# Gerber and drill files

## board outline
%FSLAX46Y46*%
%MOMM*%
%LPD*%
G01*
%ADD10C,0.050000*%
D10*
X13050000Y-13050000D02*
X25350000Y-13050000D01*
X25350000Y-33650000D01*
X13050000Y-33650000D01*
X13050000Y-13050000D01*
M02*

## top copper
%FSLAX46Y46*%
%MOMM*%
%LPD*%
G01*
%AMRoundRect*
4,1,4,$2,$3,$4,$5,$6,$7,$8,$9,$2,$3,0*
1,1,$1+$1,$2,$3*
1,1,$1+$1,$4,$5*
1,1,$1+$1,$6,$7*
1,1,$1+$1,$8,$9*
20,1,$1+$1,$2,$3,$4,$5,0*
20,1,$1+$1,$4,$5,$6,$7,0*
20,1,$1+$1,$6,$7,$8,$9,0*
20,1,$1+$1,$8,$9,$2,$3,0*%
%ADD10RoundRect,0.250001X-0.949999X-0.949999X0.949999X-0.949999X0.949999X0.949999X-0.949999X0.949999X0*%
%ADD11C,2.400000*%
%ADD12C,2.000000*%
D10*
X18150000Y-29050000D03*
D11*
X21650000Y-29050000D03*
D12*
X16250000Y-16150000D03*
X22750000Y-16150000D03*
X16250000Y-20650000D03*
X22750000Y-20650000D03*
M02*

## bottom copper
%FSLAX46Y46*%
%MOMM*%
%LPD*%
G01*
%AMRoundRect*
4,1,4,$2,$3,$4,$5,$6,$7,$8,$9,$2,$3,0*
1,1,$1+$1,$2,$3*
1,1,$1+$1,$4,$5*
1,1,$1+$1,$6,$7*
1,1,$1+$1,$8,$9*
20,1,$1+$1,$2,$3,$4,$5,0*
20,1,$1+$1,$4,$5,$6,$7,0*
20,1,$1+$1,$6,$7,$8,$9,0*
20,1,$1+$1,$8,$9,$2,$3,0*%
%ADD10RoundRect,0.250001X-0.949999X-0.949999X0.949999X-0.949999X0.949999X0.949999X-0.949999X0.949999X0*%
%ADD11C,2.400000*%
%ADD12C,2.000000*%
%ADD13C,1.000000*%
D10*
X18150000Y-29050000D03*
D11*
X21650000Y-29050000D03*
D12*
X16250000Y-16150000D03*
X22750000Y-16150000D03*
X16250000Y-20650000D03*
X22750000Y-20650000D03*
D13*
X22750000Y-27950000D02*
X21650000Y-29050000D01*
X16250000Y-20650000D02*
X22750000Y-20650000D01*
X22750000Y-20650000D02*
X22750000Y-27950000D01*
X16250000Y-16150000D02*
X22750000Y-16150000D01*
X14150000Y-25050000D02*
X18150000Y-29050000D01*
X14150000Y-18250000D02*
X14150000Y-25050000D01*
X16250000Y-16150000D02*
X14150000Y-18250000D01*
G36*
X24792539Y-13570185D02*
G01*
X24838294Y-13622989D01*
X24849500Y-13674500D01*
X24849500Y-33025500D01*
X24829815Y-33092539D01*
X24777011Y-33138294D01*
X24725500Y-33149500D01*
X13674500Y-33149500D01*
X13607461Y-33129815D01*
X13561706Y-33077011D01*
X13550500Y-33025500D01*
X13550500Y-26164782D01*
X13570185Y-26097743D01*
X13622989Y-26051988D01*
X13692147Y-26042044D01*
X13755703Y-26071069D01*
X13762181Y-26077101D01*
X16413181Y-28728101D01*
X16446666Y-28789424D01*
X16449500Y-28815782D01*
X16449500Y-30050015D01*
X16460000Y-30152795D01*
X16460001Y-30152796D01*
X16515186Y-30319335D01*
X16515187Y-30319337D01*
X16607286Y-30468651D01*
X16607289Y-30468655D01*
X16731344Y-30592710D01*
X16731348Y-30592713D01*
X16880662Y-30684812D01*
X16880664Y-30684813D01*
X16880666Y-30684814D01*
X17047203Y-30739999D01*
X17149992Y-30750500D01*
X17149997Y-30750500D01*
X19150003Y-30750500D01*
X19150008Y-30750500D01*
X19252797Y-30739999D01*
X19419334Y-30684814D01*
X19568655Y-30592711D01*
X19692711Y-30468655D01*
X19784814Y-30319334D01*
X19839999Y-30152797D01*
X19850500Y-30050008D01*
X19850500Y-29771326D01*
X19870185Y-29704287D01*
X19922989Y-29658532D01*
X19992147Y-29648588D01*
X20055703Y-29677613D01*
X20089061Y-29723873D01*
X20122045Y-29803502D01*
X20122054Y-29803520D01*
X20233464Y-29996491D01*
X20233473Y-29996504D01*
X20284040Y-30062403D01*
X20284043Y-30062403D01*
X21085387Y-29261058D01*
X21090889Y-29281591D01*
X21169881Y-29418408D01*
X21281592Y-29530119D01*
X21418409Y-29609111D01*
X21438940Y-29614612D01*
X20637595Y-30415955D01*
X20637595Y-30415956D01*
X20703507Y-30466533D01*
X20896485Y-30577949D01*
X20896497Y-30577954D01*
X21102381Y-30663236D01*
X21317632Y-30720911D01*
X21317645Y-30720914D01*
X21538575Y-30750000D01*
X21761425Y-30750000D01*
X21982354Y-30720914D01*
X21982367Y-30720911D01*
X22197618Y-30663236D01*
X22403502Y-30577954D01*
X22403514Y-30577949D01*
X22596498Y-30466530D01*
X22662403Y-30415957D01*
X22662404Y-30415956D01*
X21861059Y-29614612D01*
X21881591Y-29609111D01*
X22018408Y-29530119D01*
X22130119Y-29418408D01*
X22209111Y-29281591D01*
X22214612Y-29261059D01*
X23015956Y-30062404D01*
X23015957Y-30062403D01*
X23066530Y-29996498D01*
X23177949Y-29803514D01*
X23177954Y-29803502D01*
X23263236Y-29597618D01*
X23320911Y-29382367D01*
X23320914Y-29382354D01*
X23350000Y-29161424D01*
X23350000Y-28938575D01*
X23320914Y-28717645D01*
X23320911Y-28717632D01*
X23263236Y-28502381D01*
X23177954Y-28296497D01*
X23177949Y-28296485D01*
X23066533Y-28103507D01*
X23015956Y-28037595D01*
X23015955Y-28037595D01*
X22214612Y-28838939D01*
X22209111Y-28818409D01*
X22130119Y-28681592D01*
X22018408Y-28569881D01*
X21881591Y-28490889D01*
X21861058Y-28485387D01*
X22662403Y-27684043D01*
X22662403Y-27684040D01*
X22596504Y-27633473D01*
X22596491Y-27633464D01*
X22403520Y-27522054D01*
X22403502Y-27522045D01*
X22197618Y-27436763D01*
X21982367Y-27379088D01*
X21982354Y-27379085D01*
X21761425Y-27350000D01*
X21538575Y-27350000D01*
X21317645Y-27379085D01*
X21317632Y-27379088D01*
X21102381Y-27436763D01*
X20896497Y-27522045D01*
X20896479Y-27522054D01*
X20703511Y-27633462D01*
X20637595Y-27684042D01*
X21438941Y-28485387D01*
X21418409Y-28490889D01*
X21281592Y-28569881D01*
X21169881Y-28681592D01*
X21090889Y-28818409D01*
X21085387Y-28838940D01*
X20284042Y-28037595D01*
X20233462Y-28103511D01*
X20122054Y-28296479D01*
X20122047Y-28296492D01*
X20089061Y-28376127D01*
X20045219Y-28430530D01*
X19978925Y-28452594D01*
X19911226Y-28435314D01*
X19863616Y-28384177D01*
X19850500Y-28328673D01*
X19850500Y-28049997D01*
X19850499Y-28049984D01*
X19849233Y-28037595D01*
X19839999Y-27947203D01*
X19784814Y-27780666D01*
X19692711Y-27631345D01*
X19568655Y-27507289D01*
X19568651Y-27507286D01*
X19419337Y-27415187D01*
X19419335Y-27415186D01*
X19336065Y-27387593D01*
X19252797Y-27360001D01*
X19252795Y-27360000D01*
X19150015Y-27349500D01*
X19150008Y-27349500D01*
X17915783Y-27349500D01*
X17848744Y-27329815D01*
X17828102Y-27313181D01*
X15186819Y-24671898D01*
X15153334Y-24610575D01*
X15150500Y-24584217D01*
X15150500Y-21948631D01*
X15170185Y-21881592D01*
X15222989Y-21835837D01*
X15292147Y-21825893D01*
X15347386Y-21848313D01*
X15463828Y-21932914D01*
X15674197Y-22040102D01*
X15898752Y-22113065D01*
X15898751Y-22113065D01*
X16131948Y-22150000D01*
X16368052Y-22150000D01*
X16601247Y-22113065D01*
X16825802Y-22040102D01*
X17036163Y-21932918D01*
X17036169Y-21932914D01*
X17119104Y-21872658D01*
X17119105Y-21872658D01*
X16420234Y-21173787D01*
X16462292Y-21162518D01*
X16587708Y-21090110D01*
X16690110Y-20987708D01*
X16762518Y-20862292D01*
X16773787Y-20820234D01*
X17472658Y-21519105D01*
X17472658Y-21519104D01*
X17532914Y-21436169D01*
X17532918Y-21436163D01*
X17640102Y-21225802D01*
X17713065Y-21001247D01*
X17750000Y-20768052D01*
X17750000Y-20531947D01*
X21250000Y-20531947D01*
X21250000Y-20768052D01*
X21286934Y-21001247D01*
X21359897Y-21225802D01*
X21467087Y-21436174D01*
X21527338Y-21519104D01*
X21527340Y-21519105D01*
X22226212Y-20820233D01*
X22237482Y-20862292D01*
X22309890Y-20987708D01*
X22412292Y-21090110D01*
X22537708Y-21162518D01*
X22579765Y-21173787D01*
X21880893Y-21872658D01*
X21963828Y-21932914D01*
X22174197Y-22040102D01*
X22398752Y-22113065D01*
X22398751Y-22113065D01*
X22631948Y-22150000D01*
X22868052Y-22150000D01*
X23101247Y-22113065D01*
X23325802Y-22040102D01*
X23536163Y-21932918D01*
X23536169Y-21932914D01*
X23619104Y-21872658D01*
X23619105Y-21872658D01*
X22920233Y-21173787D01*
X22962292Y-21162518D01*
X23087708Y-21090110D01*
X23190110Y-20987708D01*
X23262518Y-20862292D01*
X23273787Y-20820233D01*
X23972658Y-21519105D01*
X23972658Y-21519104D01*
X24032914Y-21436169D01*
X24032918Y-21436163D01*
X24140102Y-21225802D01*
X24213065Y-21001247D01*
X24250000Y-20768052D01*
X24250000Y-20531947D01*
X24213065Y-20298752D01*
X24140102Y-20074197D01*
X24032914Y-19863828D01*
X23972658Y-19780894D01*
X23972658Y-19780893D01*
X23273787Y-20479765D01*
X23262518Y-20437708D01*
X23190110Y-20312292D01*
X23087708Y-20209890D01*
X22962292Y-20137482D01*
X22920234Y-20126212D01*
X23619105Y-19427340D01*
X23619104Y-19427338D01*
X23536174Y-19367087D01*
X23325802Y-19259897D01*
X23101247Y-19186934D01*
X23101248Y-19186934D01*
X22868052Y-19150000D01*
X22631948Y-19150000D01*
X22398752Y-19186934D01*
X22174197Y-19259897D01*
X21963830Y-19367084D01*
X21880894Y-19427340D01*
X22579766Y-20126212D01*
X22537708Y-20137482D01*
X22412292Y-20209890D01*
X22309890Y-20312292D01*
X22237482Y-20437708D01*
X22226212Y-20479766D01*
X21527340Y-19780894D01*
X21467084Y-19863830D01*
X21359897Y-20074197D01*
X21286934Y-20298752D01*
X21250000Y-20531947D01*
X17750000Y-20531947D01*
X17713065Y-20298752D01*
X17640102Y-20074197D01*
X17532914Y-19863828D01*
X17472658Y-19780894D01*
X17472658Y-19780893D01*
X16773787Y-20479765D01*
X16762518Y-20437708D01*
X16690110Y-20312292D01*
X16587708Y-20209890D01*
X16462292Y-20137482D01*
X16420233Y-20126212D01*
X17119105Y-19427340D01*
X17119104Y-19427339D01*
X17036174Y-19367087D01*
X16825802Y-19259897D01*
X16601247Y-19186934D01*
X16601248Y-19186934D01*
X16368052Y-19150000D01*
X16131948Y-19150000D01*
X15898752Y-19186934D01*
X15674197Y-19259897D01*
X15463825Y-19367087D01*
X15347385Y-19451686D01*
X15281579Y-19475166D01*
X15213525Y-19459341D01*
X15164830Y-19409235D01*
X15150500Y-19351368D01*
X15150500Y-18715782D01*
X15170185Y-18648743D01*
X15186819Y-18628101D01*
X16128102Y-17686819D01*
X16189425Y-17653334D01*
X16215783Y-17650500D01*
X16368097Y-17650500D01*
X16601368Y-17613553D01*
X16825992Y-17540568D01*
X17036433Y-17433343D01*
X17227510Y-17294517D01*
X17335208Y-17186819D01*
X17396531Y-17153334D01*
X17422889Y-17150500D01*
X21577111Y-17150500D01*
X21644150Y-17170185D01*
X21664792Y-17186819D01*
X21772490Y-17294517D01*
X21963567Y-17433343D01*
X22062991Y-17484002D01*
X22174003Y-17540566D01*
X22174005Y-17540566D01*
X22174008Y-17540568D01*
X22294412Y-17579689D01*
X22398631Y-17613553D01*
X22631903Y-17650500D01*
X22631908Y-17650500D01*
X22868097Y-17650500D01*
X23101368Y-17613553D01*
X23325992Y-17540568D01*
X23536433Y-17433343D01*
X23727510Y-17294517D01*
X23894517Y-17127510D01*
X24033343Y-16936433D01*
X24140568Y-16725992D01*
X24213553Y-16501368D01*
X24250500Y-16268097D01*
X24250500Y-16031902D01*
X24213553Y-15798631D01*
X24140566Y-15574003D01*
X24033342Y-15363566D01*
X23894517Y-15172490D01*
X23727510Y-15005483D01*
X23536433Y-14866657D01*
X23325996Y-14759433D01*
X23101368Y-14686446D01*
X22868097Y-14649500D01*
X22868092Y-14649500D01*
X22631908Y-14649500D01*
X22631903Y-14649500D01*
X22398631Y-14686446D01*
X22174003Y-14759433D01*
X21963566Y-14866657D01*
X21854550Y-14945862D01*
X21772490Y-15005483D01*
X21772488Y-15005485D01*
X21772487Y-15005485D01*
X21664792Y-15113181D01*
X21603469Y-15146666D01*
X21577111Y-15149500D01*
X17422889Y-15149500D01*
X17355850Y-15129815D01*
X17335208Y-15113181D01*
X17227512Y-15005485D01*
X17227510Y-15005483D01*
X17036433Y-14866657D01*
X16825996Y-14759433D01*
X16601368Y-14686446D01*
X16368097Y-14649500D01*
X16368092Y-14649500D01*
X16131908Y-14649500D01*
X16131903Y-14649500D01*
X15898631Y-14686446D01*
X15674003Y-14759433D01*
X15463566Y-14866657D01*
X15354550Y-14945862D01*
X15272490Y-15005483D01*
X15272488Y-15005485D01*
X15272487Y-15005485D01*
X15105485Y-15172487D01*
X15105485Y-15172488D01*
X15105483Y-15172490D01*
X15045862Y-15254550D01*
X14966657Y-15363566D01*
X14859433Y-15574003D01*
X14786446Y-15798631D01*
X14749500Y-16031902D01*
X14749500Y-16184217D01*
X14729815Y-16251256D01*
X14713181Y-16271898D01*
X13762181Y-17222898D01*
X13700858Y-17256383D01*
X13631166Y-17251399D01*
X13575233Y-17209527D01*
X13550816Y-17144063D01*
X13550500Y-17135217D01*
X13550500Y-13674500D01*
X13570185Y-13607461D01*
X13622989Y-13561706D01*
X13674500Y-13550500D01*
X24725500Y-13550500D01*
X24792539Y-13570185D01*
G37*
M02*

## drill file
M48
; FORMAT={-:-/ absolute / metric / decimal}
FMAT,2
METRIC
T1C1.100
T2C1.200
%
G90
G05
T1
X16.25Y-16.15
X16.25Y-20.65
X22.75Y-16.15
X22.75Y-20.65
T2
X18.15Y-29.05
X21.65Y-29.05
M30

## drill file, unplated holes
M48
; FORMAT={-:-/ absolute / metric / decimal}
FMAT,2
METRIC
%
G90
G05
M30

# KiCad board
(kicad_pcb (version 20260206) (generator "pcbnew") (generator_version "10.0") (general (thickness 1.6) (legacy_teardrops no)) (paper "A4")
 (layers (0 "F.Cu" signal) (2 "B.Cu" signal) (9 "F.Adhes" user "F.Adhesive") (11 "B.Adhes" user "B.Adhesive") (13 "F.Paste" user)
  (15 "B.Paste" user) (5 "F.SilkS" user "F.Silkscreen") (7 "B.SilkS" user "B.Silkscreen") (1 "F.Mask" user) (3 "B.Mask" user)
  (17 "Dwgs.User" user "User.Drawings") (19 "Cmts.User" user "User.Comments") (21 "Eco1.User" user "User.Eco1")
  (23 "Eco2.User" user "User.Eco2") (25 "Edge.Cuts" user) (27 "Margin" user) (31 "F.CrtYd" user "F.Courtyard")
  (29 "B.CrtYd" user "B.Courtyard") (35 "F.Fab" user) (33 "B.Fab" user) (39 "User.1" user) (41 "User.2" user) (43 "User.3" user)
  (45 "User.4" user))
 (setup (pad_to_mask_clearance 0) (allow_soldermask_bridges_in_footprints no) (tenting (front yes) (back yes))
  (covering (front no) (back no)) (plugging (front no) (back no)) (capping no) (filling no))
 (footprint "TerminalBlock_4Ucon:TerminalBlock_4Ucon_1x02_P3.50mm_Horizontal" (layer "F.Cu") (at 18.15 29.05)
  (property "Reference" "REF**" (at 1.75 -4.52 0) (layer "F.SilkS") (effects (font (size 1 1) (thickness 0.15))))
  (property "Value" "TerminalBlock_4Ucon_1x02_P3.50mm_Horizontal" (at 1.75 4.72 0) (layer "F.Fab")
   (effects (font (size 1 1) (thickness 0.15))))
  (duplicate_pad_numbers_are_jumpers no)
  (pad "1" thru_hole roundrect (at 0 0) (size 2.4 2.4) (drill 1.2) (layers "*.Cu" "*.Mask") (remove_unused_layers no)
   (roundrect_rratio 0.104167) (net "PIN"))
  (pad "2" thru_hole circle (at 3.5 0) (size 2.4 2.4) (drill 1.2) (layers "*.Cu" "*.Mask") (remove_unused_layers no) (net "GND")))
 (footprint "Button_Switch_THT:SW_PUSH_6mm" (layer "F.Cu") (at 16.25 16.15)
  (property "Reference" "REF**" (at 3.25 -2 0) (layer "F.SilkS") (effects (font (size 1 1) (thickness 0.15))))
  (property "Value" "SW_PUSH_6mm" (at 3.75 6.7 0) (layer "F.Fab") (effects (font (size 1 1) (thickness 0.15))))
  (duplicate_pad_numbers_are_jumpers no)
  (pad "1" thru_hole circle (at 0 0 90) (size 2 2) (drill 1.1) (layers "*.Cu" "*.Mask") (remove_unused_layers no) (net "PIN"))
  (pad "1" thru_hole circle (at 6.5 0 90) (size 2 2) (drill 1.1) (layers "*.Cu" "*.Mask") (remove_unused_layers no) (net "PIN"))
  (pad "2" thru_hole circle (at 0 4.5 90) (size 2 2) (drill 1.1) (layers "*.Cu" "*.Mask") (remove_unused_layers no) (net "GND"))
  (pad "2" thru_hole circle (at 6.5 4.5 90) (size 2 2) (drill 1.1) (layers "*.Cu" "*.Mask") (remove_unused_layers no) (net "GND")))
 (gr_rect (start 13.05 13.05) (end 25.35 33.65) (stroke (width 0.05) (type default)) (fill no) (layer "Edge.Cuts"))
 (segment (start 16.25 16.15) (end 22.75 16.15) (width 1) (layer "B.Cu") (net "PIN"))
 (segment (start 14.15 25.05) (end 18.15 29.05) (width 1) (layer "B.Cu") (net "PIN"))
 (segment (start 14.15 18.25) (end 14.15 25.05) (width 1) (layer "B.Cu") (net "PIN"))
 (segment (start 16.25 16.15) (end 14.15 18.25) (width 1) (layer "B.Cu") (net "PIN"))
 (segment (start 22.75 27.95) (end 21.65 29.05) (width 1) (layer "B.Cu") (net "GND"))
 (segment (start 16.25 20.65) (end 22.75 20.65) (width 1) (layer "B.Cu") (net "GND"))
 (segment (start 22.75 20.65) (end 22.75 27.95) (width 1) (layer "B.Cu") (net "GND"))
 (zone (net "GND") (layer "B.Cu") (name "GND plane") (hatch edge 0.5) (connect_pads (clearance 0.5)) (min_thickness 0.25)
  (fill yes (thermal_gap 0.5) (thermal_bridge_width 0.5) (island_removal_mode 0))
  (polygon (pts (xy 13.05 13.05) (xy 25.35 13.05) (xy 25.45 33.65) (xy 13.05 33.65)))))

